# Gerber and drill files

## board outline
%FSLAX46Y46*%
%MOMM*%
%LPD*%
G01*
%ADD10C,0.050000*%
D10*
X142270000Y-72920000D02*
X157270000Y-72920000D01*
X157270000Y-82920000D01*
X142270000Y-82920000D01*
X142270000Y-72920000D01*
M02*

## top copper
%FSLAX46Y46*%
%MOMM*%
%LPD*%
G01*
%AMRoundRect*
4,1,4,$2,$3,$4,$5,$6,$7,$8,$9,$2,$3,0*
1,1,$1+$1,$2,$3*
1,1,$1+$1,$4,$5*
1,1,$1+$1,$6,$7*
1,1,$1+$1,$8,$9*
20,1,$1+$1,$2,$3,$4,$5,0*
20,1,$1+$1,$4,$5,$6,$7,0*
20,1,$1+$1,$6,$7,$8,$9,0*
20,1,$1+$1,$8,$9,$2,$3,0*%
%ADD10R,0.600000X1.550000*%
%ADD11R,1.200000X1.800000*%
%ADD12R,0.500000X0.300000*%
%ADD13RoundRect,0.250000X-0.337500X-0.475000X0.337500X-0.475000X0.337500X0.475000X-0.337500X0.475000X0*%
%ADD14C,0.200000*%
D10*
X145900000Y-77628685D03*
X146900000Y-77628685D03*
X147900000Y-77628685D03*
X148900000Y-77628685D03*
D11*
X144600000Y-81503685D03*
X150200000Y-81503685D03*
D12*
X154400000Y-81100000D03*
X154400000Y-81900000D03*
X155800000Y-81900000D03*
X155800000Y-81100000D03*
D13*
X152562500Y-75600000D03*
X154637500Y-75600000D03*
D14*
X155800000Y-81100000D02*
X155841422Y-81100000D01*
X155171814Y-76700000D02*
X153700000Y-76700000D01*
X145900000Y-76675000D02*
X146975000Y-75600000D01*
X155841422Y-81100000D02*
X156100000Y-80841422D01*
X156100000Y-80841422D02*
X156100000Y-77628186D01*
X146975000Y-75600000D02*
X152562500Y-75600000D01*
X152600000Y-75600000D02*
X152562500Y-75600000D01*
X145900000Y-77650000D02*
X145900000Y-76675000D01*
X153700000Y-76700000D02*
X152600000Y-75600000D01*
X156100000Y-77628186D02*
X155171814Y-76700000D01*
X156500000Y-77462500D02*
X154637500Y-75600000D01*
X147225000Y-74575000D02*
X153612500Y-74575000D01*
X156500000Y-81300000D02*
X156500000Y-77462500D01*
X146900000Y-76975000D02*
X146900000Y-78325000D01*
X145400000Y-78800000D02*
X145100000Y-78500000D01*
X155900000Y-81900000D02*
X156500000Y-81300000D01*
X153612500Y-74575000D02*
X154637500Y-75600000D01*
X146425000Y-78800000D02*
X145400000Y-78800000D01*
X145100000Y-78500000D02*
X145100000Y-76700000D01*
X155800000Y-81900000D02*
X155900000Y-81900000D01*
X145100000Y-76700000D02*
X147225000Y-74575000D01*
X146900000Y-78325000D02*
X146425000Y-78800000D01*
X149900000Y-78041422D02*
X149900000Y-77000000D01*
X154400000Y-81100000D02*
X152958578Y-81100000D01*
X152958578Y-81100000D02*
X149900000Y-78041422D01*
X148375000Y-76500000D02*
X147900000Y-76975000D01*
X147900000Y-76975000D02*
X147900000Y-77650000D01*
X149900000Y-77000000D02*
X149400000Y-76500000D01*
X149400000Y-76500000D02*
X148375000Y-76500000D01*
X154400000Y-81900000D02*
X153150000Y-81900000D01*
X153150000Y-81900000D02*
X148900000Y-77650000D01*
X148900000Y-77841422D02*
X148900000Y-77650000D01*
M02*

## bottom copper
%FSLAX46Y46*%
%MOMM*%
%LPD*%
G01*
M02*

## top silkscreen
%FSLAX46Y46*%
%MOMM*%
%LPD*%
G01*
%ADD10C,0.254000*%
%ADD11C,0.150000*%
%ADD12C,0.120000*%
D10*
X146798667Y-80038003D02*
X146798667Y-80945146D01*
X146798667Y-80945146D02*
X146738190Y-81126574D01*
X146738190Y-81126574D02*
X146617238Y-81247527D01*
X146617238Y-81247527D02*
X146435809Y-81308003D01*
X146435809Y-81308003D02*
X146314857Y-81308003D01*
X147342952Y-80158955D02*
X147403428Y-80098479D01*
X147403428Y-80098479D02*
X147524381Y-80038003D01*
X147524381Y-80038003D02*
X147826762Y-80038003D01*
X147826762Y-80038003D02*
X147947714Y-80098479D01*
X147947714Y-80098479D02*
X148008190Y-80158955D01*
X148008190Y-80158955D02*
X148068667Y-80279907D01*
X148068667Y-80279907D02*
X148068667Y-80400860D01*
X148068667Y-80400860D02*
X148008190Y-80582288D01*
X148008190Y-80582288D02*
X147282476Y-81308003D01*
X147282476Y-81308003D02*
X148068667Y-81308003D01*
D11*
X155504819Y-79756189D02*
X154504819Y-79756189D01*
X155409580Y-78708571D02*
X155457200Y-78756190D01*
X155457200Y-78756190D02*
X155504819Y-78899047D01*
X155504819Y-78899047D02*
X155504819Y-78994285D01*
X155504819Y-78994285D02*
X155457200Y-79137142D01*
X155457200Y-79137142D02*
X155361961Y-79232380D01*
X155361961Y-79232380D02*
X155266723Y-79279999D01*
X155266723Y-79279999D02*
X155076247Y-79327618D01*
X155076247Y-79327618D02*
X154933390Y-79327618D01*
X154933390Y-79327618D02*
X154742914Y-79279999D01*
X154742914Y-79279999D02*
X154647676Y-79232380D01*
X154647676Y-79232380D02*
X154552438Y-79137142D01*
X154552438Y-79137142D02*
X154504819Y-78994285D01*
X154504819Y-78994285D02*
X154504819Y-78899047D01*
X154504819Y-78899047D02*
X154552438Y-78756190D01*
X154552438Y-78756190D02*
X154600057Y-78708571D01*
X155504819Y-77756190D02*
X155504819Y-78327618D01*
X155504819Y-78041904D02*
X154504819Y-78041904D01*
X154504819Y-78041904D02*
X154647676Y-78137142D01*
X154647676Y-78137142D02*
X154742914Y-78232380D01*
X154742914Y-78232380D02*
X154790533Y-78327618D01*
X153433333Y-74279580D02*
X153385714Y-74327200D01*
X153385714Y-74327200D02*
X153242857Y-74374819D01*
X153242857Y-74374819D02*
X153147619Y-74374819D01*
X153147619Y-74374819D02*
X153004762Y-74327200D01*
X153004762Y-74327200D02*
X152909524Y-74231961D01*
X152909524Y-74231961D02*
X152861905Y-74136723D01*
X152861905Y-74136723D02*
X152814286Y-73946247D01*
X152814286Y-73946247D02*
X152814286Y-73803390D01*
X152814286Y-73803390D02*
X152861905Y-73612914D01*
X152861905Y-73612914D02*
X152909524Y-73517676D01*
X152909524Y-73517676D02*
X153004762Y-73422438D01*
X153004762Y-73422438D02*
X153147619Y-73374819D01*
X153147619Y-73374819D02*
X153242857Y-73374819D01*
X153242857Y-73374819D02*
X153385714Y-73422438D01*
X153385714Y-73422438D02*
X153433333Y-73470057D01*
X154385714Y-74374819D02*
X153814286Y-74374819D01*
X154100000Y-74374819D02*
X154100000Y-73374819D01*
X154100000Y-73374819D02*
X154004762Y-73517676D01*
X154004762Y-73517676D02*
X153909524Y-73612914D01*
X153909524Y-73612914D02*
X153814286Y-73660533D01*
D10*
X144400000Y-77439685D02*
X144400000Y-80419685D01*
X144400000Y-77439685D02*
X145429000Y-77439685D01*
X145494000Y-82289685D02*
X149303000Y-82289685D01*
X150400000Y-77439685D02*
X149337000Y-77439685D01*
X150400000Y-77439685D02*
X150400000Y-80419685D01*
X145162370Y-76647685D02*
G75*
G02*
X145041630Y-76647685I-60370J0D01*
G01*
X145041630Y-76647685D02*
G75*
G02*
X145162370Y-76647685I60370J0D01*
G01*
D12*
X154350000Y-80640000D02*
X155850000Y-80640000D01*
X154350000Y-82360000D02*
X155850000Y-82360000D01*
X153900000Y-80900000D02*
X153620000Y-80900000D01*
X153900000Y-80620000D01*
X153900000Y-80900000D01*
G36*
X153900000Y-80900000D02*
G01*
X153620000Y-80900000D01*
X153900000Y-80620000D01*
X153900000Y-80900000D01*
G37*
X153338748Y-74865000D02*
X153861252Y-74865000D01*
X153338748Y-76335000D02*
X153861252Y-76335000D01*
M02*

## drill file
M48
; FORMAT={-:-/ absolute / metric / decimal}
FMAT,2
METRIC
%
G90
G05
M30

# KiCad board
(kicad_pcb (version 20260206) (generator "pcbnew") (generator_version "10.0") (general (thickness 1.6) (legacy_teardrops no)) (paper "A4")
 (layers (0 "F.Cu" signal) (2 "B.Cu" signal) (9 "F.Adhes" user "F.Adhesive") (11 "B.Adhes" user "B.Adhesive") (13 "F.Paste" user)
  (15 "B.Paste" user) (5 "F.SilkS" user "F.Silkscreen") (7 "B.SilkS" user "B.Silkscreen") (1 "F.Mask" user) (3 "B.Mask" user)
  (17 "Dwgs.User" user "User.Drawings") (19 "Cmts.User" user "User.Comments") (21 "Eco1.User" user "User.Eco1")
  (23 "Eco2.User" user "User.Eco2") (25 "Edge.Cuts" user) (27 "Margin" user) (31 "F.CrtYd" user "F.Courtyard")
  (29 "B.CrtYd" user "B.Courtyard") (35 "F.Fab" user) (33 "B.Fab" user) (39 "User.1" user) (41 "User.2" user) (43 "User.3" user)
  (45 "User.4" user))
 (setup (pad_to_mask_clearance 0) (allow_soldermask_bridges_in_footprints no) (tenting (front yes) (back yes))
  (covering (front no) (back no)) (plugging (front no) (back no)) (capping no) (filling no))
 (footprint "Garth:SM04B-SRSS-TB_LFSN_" (layer "F.Cu") (at 144.4 82.289685)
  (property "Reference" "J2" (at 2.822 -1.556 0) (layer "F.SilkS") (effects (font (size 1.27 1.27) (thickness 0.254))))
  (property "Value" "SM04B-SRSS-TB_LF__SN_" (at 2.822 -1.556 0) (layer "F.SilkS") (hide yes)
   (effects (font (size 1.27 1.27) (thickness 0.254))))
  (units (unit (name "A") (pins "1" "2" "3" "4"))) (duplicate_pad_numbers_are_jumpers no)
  (fp_line (start 0 -4.85) (end 0 -1.87) (stroke (width 0.254) (type solid)) (layer "F.SilkS"))
  (fp_line (start 0 -4.85) (end 1.029 -4.85) (stroke (width 0.254) (type solid)) (layer "F.SilkS"))
  (fp_line (start 1.094 0) (end 4.903 0) (stroke (width 0.254) (type solid)) (layer "F.SilkS"))
  (fp_line (start 6 -4.85) (end 4.937 -4.85) (stroke (width 0.254) (type solid)) (layer "F.SilkS"))
  (fp_line (start 6 -4.85) (end 6 -1.87) (stroke (width 0.254) (type solid)) (layer "F.SilkS"))
  (fp_circle (center 0.702 -5.642) (end 0.702 -5.58163) (stroke (width 0.254) (type solid)) (fill no) (layer "F.SilkS"))
  (pad "1" smd rect (at 1.5 -4.661) (size 0.6 1.55) (layers "F.Cu" "F.Mask" "F.Paste") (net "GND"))
  (pad "2" smd rect (at 2.5 -4.661) (size 0.6 1.55) (layers "F.Cu" "F.Mask" "F.Paste") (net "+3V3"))
  (pad "3" smd rect (at 3.5 -4.661) (size 0.6 1.55) (layers "F.Cu" "F.Mask" "F.Paste") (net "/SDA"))
  (pad "4" smd rect (at 4.5 -4.661) (size 0.6 1.55) (layers "F.Cu" "F.Mask" "F.Paste") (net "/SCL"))
  (pad "5" smd rect (at 0.2 -0.786) (size 1.2 1.8) (layers "F.Cu" "F.Mask" "F.Paste"))
  (pad "6" smd rect (at 5.8 -0.786) (size 1.2 1.8) (layers "F.Cu" "F.Mask" "F.Paste")))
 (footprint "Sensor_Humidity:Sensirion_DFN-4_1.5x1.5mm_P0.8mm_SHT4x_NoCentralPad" (layer "F.Cu") (at 155.1 81.5)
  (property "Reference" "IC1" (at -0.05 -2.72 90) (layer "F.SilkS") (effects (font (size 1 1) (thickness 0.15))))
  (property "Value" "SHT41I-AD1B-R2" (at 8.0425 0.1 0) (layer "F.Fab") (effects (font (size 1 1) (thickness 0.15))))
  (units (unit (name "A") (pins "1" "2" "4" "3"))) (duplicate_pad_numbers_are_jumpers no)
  (fp_line (start -0.75 -0.86) (end 0.75 -0.86) (stroke (width 0.12) (type solid)) (layer "F.SilkS"))
  (fp_line (start -0.75 0.86) (end 0.75 0.86) (stroke (width 0.12) (type solid)) (layer "F.SilkS"))
  (fp_poly
   (pts (xy -1.2 -0.6) (xy -1.48 -0.6) (xy -1.2 -0.88) (xy -1.2 -0.6)) (stroke (width 0.12) (type solid)) (fill yes) (layer "F.SilkS"))
  (pad "1" smd rect (at -0.7 -0.4) (size 0.5 0.3) (layers "F.Cu" "F.Mask" "F.Paste") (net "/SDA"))
  (pad "2" smd rect (at -0.7 0.4) (size 0.5 0.3) (layers "F.Cu" "F.Mask" "F.Paste") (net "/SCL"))
  (pad "3" smd rect (at 0.7 0.4) (size 0.5 0.3) (layers "F.Cu" "F.Mask" "F.Paste") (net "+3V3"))
  (pad "4" smd rect (at 0.7 -0.4) (size 0.5 0.3) (layers "F.Cu" "F.Mask" "F.Paste") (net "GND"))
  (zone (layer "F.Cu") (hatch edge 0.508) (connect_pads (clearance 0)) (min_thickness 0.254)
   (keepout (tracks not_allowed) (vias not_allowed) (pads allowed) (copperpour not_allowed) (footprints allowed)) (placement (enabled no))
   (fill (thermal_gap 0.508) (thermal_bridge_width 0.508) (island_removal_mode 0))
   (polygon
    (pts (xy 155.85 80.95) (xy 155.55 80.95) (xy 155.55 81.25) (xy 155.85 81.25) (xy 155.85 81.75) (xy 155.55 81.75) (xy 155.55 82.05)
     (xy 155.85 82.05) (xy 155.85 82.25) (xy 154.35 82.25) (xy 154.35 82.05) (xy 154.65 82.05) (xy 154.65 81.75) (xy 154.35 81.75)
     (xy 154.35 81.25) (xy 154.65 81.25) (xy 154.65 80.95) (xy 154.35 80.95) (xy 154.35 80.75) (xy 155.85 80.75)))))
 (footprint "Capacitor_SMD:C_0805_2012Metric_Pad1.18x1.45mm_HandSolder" (layer "F.Cu") (at 153.6 75.6)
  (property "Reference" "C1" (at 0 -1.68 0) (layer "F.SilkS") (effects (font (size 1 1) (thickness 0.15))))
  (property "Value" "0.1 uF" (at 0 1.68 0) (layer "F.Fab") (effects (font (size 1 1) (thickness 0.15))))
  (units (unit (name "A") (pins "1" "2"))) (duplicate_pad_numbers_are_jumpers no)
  (fp_line (start -0.261252 -0.735) (end 0.261252 -0.735) (stroke (width 0.12) (type solid)) (layer "F.SilkS"))
  (fp_line (start -0.261252 0.735) (end 0.261252 0.735) (stroke (width 0.12) (type solid)) (layer "F.SilkS"))
  (pad "1" smd roundrect (at -1.0375 0) (size 1.175 1.45) (layers "F.Cu" "F.Mask" "F.Paste") (roundrect_rratio 0.212766) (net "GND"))
  (pad "2" smd roundrect (at 1.0375 0) (size 1.175 1.45) (layers "F.Cu" "F.Mask" "F.Paste") (roundrect_rratio 0.212766) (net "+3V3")))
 (gr_rect (start 142.27 72.92) (end 157.27 82.92) (stroke (width 0.05) (type solid)) (fill no) (locked yes) (layer "Edge.Cuts"))
 (segment (start 155.8 81.1) (end 155.841422 81.1) (width 0.2) (layer "F.Cu") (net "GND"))
 (segment (start 155.171814 76.7) (end 153.7 76.7) (width 0.2) (layer "F.Cu") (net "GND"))
 (segment (start 145.9 76.675) (end 146.975 75.6) (width 0.2) (layer "F.Cu") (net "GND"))
 (segment (start 155.841422 81.1) (end 156.1 80.841422) (width 0.2) (layer "F.Cu") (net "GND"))
 (segment (start 156.1 80.841422) (end 156.1 77.628186) (width 0.2) (layer "F.Cu") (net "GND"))
 (segment (start 146.975 75.6) (end 152.5625 75.6) (width 0.2) (layer "F.Cu") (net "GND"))
 (segment (start 152.6 75.6) (end 152.5625 75.6) (width 0.2) (layer "F.Cu") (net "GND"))
 (segment (start 145.9 77.65) (end 145.9 76.675) (width 0.2) (layer "F.Cu") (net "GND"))
 (segment (start 153.7 76.7) (end 152.6 75.6) (width 0.2) (layer "F.Cu") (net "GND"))
 (segment (start 156.1 77.628186) (end 155.171814 76.7) (width 0.2) (layer "F.Cu") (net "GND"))
 (segment (start 156.5 77.4625) (end 154.6375 75.6) (width 0.2) (layer "F.Cu") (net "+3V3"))
 (segment (start 147.225 74.575) (end 153.6125 74.575) (width 0.2) (layer "F.Cu") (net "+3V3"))
 (segment (start 156.5 81.3) (end 156.5 77.4625) (width 0.2) (layer "F.Cu") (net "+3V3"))
 (segment (start 146.9 76.975) (end 146.9 78.325) (width 0.2) (layer "F.Cu") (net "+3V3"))
 (segment (start 145.4 78.8) (end 145.1 78.5) (width 0.2) (layer "F.Cu") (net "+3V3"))
 (segment (start 155.9 81.9) (end 156.5 81.3) (width 0.2) (layer "F.Cu") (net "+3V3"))
 (segment (start 153.6125 74.575) (end 154.6375 75.6) (width 0.2) (layer "F.Cu") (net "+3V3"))
 (segment (start 146.425 78.8) (end 145.4 78.8) (width 0.2) (layer "F.Cu") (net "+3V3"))
 (segment (start 145.1 78.5) (end 145.1 76.7) (width 0.2) (layer "F.Cu") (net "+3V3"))
 (segment (start 155.8 81.9) (end 155.9 81.9) (width 0.2) (layer "F.Cu") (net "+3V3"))
 (segment (start 145.1 76.7) (end 147.225 74.575) (width 0.2) (layer "F.Cu") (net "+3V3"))
 (segment (start 146.9 78.325) (end 146.425 78.8) (width 0.2) (layer "F.Cu") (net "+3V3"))
 (segment (start 149.9 78.041422) (end 149.9 77) (width 0.2) (layer "F.Cu") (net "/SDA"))
 (segment (start 154.4 81.1) (end 152.958578 81.1) (width 0.2) (layer "F.Cu") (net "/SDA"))
 (segment (start 152.958578 81.1) (end 149.9 78.041422) (width 0.2) (layer "F.Cu") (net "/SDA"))
 (segment (start 148.375 76.5) (end 147.9 76.975) (width 0.2) (layer "F.Cu") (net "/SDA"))
 (segment (start 147.9 76.975) (end 147.9 77.65) (width 0.2) (layer "F.Cu") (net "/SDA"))
 (segment (start 149.9 77) (end 149.4 76.5) (width 0.2) (layer "F.Cu") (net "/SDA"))
 (segment (start 149.4 76.5) (end 148.375 76.5) (width 0.2) (layer "F.Cu") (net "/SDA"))
 (segment (start 154.4 81.9) (end 153.15 81.9) (width 0.2) (layer "F.Cu") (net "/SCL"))
 (segment (start 153.15 81.9) (end 148.9 77.65) (width 0.2) (layer "F.Cu") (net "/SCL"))
 (segment (start 148.9 77.841422) (end 148.9 77.65) (width 0.2) (layer "F.Cu") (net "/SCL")))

